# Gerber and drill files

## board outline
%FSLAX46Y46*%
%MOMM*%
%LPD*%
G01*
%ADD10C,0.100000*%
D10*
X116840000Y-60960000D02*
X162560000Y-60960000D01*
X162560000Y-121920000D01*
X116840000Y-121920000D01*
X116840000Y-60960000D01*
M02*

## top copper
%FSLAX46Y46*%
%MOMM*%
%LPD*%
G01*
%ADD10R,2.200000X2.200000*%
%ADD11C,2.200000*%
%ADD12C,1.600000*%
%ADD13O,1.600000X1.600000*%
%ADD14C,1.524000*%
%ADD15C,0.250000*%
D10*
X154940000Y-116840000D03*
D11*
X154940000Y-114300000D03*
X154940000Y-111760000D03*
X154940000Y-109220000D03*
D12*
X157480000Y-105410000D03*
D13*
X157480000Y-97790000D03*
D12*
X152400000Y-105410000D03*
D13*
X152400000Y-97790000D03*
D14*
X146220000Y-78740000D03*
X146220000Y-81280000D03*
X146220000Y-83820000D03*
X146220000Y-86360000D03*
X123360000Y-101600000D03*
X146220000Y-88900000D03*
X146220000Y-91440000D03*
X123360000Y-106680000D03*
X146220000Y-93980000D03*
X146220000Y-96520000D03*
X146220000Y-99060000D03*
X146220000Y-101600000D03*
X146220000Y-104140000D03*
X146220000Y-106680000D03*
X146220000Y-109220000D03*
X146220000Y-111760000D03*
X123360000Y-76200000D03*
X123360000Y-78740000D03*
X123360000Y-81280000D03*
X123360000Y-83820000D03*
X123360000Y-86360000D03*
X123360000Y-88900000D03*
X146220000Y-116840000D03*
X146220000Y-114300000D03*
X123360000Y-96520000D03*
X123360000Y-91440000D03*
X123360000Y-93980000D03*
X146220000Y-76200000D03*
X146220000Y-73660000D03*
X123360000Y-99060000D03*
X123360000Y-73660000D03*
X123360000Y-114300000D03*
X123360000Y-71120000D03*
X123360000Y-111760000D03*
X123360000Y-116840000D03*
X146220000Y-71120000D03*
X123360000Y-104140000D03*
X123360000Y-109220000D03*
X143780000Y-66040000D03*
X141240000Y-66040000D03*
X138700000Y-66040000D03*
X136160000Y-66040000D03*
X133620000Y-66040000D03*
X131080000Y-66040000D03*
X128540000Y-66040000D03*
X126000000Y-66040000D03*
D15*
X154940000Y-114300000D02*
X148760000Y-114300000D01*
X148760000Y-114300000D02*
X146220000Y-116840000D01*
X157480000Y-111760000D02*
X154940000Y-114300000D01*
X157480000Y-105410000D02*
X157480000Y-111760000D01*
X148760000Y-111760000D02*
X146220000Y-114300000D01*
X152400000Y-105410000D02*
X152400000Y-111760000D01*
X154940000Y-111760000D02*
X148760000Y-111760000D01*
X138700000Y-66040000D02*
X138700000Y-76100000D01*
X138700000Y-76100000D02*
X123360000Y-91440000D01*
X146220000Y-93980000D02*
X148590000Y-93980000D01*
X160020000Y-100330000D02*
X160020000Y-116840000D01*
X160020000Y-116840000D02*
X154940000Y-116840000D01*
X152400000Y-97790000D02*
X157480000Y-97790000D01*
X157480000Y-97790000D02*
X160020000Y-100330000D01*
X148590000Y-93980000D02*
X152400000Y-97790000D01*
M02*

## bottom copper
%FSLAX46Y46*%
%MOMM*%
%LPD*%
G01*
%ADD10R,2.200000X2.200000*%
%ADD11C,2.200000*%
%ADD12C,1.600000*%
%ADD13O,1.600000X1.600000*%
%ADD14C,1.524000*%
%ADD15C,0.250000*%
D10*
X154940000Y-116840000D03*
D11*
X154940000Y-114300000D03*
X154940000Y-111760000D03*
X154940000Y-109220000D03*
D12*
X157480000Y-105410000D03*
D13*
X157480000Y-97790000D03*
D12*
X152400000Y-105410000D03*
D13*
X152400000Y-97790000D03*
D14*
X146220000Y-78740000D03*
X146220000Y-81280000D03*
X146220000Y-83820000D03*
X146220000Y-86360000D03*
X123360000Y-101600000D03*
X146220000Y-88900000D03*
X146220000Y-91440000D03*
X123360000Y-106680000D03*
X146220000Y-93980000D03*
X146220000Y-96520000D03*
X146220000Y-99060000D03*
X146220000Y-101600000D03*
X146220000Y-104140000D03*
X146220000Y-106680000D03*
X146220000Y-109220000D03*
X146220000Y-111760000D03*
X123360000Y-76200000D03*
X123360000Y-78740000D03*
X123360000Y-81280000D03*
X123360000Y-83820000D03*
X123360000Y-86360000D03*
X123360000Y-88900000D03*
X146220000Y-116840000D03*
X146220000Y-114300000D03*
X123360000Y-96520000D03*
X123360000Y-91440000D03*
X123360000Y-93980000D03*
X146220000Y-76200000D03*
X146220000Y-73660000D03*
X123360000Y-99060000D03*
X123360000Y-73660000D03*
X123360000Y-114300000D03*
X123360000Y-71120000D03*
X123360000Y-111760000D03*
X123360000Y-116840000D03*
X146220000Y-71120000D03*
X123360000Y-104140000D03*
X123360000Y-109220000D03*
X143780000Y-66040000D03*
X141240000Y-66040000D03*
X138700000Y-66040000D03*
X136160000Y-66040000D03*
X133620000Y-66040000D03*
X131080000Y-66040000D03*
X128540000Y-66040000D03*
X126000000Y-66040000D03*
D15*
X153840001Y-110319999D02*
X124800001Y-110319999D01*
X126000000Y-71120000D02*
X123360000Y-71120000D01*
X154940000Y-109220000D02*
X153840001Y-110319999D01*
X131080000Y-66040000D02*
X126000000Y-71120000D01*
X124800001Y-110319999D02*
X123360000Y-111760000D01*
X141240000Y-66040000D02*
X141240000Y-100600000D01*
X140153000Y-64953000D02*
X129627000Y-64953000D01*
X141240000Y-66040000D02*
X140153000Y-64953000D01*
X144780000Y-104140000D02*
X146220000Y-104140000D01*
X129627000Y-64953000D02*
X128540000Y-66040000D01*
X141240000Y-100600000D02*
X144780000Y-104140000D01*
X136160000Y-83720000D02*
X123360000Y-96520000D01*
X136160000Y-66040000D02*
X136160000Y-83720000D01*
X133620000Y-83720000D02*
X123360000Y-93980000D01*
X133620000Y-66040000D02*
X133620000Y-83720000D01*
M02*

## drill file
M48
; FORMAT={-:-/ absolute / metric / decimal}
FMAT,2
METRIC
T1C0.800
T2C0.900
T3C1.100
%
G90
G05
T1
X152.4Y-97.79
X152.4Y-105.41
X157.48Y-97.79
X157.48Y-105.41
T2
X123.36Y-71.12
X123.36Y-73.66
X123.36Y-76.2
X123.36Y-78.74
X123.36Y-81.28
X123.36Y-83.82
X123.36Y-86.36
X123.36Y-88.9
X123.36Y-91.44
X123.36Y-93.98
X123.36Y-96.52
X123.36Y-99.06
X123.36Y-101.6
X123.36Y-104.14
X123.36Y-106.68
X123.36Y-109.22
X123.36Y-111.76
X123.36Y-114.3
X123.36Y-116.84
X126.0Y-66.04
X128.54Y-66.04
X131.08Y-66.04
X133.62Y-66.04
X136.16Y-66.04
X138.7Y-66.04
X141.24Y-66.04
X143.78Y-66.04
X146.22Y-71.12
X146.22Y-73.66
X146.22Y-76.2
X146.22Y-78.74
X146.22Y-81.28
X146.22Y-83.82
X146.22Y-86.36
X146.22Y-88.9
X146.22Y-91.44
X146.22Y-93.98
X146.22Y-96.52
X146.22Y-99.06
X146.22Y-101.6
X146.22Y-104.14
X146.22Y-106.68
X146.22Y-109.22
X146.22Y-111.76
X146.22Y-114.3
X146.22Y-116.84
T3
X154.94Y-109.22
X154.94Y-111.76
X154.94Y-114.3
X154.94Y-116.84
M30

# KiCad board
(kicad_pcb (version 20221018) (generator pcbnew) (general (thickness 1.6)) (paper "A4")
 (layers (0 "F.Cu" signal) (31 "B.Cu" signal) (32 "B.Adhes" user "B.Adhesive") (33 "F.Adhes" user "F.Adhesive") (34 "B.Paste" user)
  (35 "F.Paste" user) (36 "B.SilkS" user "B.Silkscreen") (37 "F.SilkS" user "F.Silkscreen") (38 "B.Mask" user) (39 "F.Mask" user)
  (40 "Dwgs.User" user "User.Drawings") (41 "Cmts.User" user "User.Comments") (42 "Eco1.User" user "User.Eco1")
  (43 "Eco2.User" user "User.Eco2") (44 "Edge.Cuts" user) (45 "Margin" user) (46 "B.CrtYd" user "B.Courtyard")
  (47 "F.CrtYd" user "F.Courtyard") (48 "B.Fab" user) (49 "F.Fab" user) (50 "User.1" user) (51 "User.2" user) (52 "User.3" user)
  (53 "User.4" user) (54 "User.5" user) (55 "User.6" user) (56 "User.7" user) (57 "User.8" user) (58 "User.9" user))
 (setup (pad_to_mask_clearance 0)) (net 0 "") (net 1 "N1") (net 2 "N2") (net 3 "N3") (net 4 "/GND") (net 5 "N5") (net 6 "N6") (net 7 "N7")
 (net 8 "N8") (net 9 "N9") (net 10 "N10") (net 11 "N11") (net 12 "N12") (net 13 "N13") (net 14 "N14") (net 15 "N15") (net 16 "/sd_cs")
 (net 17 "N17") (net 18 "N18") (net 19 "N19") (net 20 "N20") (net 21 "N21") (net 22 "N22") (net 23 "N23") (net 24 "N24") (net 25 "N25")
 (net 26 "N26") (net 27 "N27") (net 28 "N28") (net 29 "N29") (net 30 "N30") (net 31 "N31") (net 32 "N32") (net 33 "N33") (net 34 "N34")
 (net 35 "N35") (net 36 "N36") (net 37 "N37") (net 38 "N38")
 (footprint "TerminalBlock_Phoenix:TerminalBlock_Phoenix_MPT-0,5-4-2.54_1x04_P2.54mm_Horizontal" (layer "F.Cu") (at 154.94 116.84 90)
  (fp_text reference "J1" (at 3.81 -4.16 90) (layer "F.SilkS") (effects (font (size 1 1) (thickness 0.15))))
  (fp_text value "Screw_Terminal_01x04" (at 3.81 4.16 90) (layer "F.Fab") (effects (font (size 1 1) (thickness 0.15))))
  (pad "1" thru_hole rect (at 0 0 90) (size 2.2 2.2) (drill 1.1) (layers "*.Cu" "*.Mask") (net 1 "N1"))
  (pad "2" thru_hole circle (at 2.54 0 90) (size 2.2 2.2) (drill 1.1) (layers "*.Cu" "*.Mask") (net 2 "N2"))
  (pad "3" thru_hole circle (at 5.08 0 90) (size 2.2 2.2) (drill 1.1) (layers "*.Cu" "*.Mask") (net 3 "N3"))
  (pad "4" thru_hole circle (at 7.62 0 90) (size 2.2 2.2) (drill 1.1) (layers "*.Cu" "*.Mask") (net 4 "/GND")))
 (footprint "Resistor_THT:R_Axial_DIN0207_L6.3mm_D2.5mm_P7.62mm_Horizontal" (layer "F.Cu") (at 157.48 105.41 90)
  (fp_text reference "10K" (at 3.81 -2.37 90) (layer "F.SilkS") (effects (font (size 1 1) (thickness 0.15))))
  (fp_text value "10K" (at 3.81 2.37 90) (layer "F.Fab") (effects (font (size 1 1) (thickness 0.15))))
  (pad "1" thru_hole circle (at 0 0 90) (size 1.6 1.6) (drill 0.8) (layers "*.Cu" "*.Mask") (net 2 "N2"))
  (pad "2" thru_hole oval (at 7.62 0 90) (size 1.6 1.6) (drill 0.8) (layers "*.Cu" "*.Mask") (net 1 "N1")))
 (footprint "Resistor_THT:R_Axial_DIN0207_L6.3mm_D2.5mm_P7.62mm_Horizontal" (layer "F.Cu") (at 152.4 105.41 90)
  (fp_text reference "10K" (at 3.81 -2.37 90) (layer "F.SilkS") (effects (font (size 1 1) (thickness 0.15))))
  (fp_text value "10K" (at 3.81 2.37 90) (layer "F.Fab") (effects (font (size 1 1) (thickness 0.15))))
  (pad "1" thru_hole circle (at 0 0 90) (size 1.6 1.6) (drill 0.8) (layers "*.Cu" "*.Mask") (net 3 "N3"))
  (pad "2" thru_hole oval (at 7.62 0 90) (size 1.6 1.6) (drill 0.8) (layers "*.Cu" "*.Mask") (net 1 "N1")))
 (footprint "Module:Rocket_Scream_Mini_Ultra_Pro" (layer "F.Cu") (at 136.06 93.98)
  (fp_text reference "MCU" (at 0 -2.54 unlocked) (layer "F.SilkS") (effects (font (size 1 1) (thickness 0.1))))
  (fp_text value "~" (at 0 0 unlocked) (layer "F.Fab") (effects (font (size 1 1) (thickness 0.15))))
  (pad "0" thru_hole circle (at 10.16 -15.24) (size 1.524 1.524) (drill 0.9) (layers "*.Cu" "*.Mask") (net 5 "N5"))
  (pad "1" thru_hole circle (at 10.16 -12.7) (size 1.524 1.524) (drill 0.9) (layers "*.Cu" "*.Mask") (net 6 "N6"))
  (pad "2" thru_hole circle (at 10.16 -10.16) (size 1.524 1.524) (drill 0.9) (layers "*.Cu" "*.Mask") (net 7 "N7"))
  (pad "3" thru_hole circle (at 10.16 -7.62) (size 1.524 1.524) (drill 0.9) (layers "*.Cu" "*.Mask") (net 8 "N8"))
  (pad "3V3" thru_hole circle (at -12.7 7.62) (size 1.524 1.524) (drill 0.9) (layers "*.Cu" "*.Mask") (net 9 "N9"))
  (pad "4" thru_hole circle (at 10.16 -5.08) (size 1.524 1.524) (drill 0.9) (layers "*.Cu" "*.Mask") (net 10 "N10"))
  (pad "5" thru_hole circle (at 10.16 -2.54) (size 1.524 1.524) (drill 0.9) (layers "*.Cu" "*.Mask") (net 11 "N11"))
  (pad "5V" thru_hole circle (at -12.7 12.7) (size 1.524 1.524) (drill 0.9) (layers "*.Cu" "*.Mask") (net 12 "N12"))
  (pad "6" thru_hole circle (at 10.16 0) (size 1.524 1.524) (drill 0.9) (layers "*.Cu" "*.Mask") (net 1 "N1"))
  (pad "7" thru_hole circle (at 10.16 2.54) (size 1.524 1.524) (drill 0.9) (layers "*.Cu" "*.Mask") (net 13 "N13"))
  (pad "8" thru_hole circle (at 10.16 5.08) (size 1.524 1.524) (drill 0.9) (layers "*.Cu" "*.Mask") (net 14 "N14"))
  (pad "9" thru_hole circle (at 10.16 7.62) (size 1.524 1.524) (drill 0.9) (layers "*.Cu" "*.Mask") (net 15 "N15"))
  (pad "10" thru_hole circle (at 10.16 10.16) (size 1.524 1.524) (drill 0.9) (layers "*.Cu" "*.Mask") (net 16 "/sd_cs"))
  (pad "11" thru_hole circle (at 10.16 12.7) (size 1.524 1.524) (drill 0.9) (layers "*.Cu" "*.Mask") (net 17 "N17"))
  (pad "12" thru_hole circle (at 10.16 15.24) (size 1.524 1.524) (drill 0.9) (layers "*.Cu" "*.Mask") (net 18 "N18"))
  (pad "13" thru_hole circle (at 10.16 17.78) (size 1.524 1.524) (drill 0.9) (layers "*.Cu" "*.Mask") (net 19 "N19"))
  (pad "14" thru_hole circle (at -12.7 -17.78) (size 1.524 1.524) (drill 0.9) (layers "*.Cu" "*.Mask") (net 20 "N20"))
  (pad "15" thru_hole circle (at -12.7 -15.24) (size 1.524 1.524) (drill 0.9) (layers "*.Cu" "*.Mask") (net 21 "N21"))
  (pad "16" thru_hole circle (at -12.7 -12.7) (size 1.524 1.524) (drill 0.9) (layers "*.Cu" "*.Mask") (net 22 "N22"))
  (pad "17" thru_hole circle (at -12.7 -10.16) (size 1.524 1.524) (drill 0.9) (layers "*.Cu" "*.Mask") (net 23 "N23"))
  (pad "18" thru_hole circle (at -12.7 -7.62) (size 1.524 1.524) (drill 0.9) (layers "*.Cu" "*.Mask") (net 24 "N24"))
  (pad "19" thru_hole circle (at -12.7 -5.08) (size 1.524 1.524) (drill 0.9) (layers "*.Cu" "*.Mask") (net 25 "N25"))
  (pad "20" thru_hole circle (at 10.16 22.86) (size 1.524 1.524) (drill 0.9) (layers "*.Cu" "*.Mask") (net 2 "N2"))
  (pad "21" thru_hole circle (at 10.16 20.32) (size 1.524 1.524) (drill 0.9) (layers "*.Cu" "*.Mask") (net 3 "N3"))
  (pad "22" thru_hole circle (at -12.7 2.54) (size 1.524 1.524) (drill 0.9) (layers "*.Cu" "*.Mask") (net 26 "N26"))
  (pad "23" thru_hole circle (at -12.7 -2.54) (size 1.524 1.524) (drill 0.9) (layers "*.Cu" "*.Mask") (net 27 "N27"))
  (pad "24" thru_hole circle (at -12.7 0) (size 1.524 1.524) (drill 0.9) (layers "*.Cu" "*.Mask") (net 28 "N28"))
  (pad "30" thru_hole circle (at 10.16 -17.78) (size 1.524 1.524) (drill 0.9) (layers "*.Cu" "*.Mask") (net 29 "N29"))
  (pad "31" thru_hole circle (at 10.16 -20.32) (size 1.524 1.524) (drill 0.9) (layers "*.Cu" "*.Mask") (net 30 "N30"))
  (pad "38" thru_hole circle (at -12.7 5.08) (size 1.524 1.524) (drill 0.9) (layers "*.Cu" "*.Mask") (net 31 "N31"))
  (pad "AREF" thru_hole circle (at -12.7 -20.32) (size 1.524 1.524) (drill 0.9) (layers "*.Cu" "*.Mask") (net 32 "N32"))
  (pad "BAT" thru_hole circle (at -12.7 20.32) (size 1.524 1.524) (drill 0.9) (layers "*.Cu" "*.Mask") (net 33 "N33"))
  (pad "GND" thru_hole circle (at -12.7 -22.86) (size 1.524 1.524) (drill 0.9) (layers "*.Cu" "*.Mask") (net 4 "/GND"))
  (pad "GND" thru_hole circle (at -12.7 17.78) (size 1.524 1.524) (drill 0.9) (layers "*.Cu" "*.Mask") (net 4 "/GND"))
  (pad "GND" thru_hole circle (at -12.7 22.86) (size 1.524 1.524) (drill 0.9) (layers "*.Cu" "*.Mask") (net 4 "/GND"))
  (pad "RST" thru_hole circle (at 10.16 -22.86) (size 1.524 1.524) (drill 0.9) (layers "*.Cu" "*.Mask") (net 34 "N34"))
  (pad "VBUS" thru_hole circle (at -12.7 10.16) (size 1.524 1.524) (drill 0.9) (layers "*.Cu" "*.Mask") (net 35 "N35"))
  (pad "VIN" thru_hole circle (at -12.7 15.24) (size 1.524 1.524) (drill 0.9) (layers "*.Cu" "*.Mask") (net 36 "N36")))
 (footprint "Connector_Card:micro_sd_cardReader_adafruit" (layer "B.Cu") (at 134.12 78.74 90)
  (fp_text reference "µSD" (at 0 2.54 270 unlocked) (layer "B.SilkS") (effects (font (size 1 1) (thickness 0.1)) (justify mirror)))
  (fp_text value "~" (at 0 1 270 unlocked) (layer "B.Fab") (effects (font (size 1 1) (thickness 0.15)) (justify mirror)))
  (pad "1" thru_hole circle (at 12.7 9.66 90) (size 1.524 1.524) (drill 0.9) (layers "*.Cu" "*.Mask") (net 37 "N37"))
  (pad "2" thru_hole circle (at 12.7 7.12 90) (size 1.524 1.524) (drill 0.9) (layers "*.Cu" "*.Mask") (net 16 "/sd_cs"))
  (pad "3" thru_hole circle (at 12.7 4.58 90) (size 1.524 1.524) (drill 0.9) (layers "*.Cu" "*.Mask") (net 27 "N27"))
  (pad "4" thru_hole circle (at 12.7 2.04 90) (size 1.524 1.524) (drill 0.9) (layers "*.Cu" "*.Mask") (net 26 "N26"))
  (pad "5" thru_hole circle (at 12.7 -0.5 90) (size 1.524 1.524) (drill 0.9) (layers "*.Cu" "*.Mask") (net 28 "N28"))
  (pad "6" thru_hole circle (at 12.7 -3.04 90) (size 1.524 1.524) (drill 0.9) (layers "*.Cu" "*.Mask") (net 4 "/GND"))
  (pad "7" thru_hole circle (at 12.7 -5.58 90) (size 1.524 1.524) (drill 0.9) (layers "*.Cu" "*.Mask") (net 16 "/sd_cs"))
  (pad "8" thru_hole circle (at 12.7 -8.12 90) (size 1.524 1.524) (drill 0.9) (layers "*.Cu" "*.Mask") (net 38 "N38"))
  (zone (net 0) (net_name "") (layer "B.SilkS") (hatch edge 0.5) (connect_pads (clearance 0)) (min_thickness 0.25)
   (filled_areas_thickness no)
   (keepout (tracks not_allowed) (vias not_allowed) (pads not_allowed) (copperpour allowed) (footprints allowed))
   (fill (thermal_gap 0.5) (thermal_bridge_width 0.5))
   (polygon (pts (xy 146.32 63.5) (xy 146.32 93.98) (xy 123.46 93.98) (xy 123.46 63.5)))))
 (gr_rect (start 116.84 60.96) (end 162.56 121.92) (stroke (width 0.1) (type default)) (fill none) (layer "Edge.Cuts"))
 (segment (start 154.94 114.3) (end 148.76 114.3) (width 0.25) (layer "F.Cu") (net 2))
 (segment (start 148.76 114.3) (end 146.22 116.84) (width 0.25) (layer "F.Cu") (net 2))
 (segment (start 157.48 111.76) (end 154.94 114.3) (width 0.25) (layer "F.Cu") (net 2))
 (segment (start 157.48 105.41) (end 157.48 111.76) (width 0.25) (layer "F.Cu") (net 2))
 (segment (start 148.76 111.76) (end 146.22 114.3) (width 0.25) (layer "F.Cu") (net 3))
 (segment (start 152.4 105.41) (end 152.4 111.76) (width 0.25) (layer "F.Cu") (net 3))
 (segment (start 154.94 111.76) (end 148.76 111.76) (width 0.25) (layer "F.Cu") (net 3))
 (segment (start 153.840001 110.319999) (end 124.800001 110.319999) (width 0.25) (layer "B.Cu") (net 4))
 (segment (start 126 71.12) (end 123.36 71.12) (width 0.25) (layer "B.Cu") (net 4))
 (segment (start 154.94 109.22) (end 153.840001 110.319999) (width 0.25) (layer "B.Cu") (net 4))
 (segment (start 131.08 66.04) (end 126 71.12) (width 0.25) (layer "B.Cu") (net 4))
 (segment (start 124.800001 110.319999) (end 123.36 111.76) (width 0.25) (layer "B.Cu") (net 4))
 (segment (start 141.24 66.04) (end 141.24 100.6) (width 0.25) (layer "B.Cu") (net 16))
 (segment (start 140.153 64.953) (end 129.627 64.953) (width 0.25) (layer "B.Cu") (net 16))
 (segment (start 141.24 66.04) (end 140.153 64.953) (width 0.25) (layer "B.Cu") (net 16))
 (segment (start 144.78 104.14) (end 146.22 104.14) (width 0.25) (layer "B.Cu") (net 16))
 (segment (start 129.627 64.953) (end 128.54 66.04) (width 0.25) (layer "B.Cu") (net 16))
 (segment (start 141.24 100.6) (end 144.78 104.14) (width 0.25) (layer "B.Cu") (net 16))
 (segment (start 136.16 83.72) (end 123.36 96.52) (width 0.25) (layer "B.Cu") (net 26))
 (segment (start 136.16 66.04) (end 136.16 83.72) (width 0.25) (layer "B.Cu") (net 26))
 (segment (start 138.7 66.04) (end 138.7 76.1) (width 0.25) (layer "F.Cu") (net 27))
 (segment (start 138.7 76.1) (end 123.36 91.44) (width 0.25) (layer "F.Cu") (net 27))
 (segment (start 133.62 83.72) (end 123.36 93.98) (width 0.25) (layer "B.Cu") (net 28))
 (segment (start 133.62 66.04) (end 133.62 83.72) (width 0.25) (layer "B.Cu") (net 28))
 (segment (start 146.22 93.98) (end 148.59 93.98) (width 0.25) (layer "F.Cu") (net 1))
 (segment (start 160.02 100.33) (end 160.02 116.84) (width 0.25) (layer "F.Cu") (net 1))
 (segment (start 160.02 116.84) (end 154.94 116.84) (width 0.25) (layer "F.Cu") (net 1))
 (segment (start 152.4 97.79) (end 157.48 97.79) (width 0.25) (layer "F.Cu") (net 1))
 (segment (start 157.48 97.79) (end 160.02 100.33) (width 0.25) (layer "F.Cu") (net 1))
 (segment (start 148.59 93.98) (end 152.4 97.79) (width 0.25) (layer "F.Cu") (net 1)))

